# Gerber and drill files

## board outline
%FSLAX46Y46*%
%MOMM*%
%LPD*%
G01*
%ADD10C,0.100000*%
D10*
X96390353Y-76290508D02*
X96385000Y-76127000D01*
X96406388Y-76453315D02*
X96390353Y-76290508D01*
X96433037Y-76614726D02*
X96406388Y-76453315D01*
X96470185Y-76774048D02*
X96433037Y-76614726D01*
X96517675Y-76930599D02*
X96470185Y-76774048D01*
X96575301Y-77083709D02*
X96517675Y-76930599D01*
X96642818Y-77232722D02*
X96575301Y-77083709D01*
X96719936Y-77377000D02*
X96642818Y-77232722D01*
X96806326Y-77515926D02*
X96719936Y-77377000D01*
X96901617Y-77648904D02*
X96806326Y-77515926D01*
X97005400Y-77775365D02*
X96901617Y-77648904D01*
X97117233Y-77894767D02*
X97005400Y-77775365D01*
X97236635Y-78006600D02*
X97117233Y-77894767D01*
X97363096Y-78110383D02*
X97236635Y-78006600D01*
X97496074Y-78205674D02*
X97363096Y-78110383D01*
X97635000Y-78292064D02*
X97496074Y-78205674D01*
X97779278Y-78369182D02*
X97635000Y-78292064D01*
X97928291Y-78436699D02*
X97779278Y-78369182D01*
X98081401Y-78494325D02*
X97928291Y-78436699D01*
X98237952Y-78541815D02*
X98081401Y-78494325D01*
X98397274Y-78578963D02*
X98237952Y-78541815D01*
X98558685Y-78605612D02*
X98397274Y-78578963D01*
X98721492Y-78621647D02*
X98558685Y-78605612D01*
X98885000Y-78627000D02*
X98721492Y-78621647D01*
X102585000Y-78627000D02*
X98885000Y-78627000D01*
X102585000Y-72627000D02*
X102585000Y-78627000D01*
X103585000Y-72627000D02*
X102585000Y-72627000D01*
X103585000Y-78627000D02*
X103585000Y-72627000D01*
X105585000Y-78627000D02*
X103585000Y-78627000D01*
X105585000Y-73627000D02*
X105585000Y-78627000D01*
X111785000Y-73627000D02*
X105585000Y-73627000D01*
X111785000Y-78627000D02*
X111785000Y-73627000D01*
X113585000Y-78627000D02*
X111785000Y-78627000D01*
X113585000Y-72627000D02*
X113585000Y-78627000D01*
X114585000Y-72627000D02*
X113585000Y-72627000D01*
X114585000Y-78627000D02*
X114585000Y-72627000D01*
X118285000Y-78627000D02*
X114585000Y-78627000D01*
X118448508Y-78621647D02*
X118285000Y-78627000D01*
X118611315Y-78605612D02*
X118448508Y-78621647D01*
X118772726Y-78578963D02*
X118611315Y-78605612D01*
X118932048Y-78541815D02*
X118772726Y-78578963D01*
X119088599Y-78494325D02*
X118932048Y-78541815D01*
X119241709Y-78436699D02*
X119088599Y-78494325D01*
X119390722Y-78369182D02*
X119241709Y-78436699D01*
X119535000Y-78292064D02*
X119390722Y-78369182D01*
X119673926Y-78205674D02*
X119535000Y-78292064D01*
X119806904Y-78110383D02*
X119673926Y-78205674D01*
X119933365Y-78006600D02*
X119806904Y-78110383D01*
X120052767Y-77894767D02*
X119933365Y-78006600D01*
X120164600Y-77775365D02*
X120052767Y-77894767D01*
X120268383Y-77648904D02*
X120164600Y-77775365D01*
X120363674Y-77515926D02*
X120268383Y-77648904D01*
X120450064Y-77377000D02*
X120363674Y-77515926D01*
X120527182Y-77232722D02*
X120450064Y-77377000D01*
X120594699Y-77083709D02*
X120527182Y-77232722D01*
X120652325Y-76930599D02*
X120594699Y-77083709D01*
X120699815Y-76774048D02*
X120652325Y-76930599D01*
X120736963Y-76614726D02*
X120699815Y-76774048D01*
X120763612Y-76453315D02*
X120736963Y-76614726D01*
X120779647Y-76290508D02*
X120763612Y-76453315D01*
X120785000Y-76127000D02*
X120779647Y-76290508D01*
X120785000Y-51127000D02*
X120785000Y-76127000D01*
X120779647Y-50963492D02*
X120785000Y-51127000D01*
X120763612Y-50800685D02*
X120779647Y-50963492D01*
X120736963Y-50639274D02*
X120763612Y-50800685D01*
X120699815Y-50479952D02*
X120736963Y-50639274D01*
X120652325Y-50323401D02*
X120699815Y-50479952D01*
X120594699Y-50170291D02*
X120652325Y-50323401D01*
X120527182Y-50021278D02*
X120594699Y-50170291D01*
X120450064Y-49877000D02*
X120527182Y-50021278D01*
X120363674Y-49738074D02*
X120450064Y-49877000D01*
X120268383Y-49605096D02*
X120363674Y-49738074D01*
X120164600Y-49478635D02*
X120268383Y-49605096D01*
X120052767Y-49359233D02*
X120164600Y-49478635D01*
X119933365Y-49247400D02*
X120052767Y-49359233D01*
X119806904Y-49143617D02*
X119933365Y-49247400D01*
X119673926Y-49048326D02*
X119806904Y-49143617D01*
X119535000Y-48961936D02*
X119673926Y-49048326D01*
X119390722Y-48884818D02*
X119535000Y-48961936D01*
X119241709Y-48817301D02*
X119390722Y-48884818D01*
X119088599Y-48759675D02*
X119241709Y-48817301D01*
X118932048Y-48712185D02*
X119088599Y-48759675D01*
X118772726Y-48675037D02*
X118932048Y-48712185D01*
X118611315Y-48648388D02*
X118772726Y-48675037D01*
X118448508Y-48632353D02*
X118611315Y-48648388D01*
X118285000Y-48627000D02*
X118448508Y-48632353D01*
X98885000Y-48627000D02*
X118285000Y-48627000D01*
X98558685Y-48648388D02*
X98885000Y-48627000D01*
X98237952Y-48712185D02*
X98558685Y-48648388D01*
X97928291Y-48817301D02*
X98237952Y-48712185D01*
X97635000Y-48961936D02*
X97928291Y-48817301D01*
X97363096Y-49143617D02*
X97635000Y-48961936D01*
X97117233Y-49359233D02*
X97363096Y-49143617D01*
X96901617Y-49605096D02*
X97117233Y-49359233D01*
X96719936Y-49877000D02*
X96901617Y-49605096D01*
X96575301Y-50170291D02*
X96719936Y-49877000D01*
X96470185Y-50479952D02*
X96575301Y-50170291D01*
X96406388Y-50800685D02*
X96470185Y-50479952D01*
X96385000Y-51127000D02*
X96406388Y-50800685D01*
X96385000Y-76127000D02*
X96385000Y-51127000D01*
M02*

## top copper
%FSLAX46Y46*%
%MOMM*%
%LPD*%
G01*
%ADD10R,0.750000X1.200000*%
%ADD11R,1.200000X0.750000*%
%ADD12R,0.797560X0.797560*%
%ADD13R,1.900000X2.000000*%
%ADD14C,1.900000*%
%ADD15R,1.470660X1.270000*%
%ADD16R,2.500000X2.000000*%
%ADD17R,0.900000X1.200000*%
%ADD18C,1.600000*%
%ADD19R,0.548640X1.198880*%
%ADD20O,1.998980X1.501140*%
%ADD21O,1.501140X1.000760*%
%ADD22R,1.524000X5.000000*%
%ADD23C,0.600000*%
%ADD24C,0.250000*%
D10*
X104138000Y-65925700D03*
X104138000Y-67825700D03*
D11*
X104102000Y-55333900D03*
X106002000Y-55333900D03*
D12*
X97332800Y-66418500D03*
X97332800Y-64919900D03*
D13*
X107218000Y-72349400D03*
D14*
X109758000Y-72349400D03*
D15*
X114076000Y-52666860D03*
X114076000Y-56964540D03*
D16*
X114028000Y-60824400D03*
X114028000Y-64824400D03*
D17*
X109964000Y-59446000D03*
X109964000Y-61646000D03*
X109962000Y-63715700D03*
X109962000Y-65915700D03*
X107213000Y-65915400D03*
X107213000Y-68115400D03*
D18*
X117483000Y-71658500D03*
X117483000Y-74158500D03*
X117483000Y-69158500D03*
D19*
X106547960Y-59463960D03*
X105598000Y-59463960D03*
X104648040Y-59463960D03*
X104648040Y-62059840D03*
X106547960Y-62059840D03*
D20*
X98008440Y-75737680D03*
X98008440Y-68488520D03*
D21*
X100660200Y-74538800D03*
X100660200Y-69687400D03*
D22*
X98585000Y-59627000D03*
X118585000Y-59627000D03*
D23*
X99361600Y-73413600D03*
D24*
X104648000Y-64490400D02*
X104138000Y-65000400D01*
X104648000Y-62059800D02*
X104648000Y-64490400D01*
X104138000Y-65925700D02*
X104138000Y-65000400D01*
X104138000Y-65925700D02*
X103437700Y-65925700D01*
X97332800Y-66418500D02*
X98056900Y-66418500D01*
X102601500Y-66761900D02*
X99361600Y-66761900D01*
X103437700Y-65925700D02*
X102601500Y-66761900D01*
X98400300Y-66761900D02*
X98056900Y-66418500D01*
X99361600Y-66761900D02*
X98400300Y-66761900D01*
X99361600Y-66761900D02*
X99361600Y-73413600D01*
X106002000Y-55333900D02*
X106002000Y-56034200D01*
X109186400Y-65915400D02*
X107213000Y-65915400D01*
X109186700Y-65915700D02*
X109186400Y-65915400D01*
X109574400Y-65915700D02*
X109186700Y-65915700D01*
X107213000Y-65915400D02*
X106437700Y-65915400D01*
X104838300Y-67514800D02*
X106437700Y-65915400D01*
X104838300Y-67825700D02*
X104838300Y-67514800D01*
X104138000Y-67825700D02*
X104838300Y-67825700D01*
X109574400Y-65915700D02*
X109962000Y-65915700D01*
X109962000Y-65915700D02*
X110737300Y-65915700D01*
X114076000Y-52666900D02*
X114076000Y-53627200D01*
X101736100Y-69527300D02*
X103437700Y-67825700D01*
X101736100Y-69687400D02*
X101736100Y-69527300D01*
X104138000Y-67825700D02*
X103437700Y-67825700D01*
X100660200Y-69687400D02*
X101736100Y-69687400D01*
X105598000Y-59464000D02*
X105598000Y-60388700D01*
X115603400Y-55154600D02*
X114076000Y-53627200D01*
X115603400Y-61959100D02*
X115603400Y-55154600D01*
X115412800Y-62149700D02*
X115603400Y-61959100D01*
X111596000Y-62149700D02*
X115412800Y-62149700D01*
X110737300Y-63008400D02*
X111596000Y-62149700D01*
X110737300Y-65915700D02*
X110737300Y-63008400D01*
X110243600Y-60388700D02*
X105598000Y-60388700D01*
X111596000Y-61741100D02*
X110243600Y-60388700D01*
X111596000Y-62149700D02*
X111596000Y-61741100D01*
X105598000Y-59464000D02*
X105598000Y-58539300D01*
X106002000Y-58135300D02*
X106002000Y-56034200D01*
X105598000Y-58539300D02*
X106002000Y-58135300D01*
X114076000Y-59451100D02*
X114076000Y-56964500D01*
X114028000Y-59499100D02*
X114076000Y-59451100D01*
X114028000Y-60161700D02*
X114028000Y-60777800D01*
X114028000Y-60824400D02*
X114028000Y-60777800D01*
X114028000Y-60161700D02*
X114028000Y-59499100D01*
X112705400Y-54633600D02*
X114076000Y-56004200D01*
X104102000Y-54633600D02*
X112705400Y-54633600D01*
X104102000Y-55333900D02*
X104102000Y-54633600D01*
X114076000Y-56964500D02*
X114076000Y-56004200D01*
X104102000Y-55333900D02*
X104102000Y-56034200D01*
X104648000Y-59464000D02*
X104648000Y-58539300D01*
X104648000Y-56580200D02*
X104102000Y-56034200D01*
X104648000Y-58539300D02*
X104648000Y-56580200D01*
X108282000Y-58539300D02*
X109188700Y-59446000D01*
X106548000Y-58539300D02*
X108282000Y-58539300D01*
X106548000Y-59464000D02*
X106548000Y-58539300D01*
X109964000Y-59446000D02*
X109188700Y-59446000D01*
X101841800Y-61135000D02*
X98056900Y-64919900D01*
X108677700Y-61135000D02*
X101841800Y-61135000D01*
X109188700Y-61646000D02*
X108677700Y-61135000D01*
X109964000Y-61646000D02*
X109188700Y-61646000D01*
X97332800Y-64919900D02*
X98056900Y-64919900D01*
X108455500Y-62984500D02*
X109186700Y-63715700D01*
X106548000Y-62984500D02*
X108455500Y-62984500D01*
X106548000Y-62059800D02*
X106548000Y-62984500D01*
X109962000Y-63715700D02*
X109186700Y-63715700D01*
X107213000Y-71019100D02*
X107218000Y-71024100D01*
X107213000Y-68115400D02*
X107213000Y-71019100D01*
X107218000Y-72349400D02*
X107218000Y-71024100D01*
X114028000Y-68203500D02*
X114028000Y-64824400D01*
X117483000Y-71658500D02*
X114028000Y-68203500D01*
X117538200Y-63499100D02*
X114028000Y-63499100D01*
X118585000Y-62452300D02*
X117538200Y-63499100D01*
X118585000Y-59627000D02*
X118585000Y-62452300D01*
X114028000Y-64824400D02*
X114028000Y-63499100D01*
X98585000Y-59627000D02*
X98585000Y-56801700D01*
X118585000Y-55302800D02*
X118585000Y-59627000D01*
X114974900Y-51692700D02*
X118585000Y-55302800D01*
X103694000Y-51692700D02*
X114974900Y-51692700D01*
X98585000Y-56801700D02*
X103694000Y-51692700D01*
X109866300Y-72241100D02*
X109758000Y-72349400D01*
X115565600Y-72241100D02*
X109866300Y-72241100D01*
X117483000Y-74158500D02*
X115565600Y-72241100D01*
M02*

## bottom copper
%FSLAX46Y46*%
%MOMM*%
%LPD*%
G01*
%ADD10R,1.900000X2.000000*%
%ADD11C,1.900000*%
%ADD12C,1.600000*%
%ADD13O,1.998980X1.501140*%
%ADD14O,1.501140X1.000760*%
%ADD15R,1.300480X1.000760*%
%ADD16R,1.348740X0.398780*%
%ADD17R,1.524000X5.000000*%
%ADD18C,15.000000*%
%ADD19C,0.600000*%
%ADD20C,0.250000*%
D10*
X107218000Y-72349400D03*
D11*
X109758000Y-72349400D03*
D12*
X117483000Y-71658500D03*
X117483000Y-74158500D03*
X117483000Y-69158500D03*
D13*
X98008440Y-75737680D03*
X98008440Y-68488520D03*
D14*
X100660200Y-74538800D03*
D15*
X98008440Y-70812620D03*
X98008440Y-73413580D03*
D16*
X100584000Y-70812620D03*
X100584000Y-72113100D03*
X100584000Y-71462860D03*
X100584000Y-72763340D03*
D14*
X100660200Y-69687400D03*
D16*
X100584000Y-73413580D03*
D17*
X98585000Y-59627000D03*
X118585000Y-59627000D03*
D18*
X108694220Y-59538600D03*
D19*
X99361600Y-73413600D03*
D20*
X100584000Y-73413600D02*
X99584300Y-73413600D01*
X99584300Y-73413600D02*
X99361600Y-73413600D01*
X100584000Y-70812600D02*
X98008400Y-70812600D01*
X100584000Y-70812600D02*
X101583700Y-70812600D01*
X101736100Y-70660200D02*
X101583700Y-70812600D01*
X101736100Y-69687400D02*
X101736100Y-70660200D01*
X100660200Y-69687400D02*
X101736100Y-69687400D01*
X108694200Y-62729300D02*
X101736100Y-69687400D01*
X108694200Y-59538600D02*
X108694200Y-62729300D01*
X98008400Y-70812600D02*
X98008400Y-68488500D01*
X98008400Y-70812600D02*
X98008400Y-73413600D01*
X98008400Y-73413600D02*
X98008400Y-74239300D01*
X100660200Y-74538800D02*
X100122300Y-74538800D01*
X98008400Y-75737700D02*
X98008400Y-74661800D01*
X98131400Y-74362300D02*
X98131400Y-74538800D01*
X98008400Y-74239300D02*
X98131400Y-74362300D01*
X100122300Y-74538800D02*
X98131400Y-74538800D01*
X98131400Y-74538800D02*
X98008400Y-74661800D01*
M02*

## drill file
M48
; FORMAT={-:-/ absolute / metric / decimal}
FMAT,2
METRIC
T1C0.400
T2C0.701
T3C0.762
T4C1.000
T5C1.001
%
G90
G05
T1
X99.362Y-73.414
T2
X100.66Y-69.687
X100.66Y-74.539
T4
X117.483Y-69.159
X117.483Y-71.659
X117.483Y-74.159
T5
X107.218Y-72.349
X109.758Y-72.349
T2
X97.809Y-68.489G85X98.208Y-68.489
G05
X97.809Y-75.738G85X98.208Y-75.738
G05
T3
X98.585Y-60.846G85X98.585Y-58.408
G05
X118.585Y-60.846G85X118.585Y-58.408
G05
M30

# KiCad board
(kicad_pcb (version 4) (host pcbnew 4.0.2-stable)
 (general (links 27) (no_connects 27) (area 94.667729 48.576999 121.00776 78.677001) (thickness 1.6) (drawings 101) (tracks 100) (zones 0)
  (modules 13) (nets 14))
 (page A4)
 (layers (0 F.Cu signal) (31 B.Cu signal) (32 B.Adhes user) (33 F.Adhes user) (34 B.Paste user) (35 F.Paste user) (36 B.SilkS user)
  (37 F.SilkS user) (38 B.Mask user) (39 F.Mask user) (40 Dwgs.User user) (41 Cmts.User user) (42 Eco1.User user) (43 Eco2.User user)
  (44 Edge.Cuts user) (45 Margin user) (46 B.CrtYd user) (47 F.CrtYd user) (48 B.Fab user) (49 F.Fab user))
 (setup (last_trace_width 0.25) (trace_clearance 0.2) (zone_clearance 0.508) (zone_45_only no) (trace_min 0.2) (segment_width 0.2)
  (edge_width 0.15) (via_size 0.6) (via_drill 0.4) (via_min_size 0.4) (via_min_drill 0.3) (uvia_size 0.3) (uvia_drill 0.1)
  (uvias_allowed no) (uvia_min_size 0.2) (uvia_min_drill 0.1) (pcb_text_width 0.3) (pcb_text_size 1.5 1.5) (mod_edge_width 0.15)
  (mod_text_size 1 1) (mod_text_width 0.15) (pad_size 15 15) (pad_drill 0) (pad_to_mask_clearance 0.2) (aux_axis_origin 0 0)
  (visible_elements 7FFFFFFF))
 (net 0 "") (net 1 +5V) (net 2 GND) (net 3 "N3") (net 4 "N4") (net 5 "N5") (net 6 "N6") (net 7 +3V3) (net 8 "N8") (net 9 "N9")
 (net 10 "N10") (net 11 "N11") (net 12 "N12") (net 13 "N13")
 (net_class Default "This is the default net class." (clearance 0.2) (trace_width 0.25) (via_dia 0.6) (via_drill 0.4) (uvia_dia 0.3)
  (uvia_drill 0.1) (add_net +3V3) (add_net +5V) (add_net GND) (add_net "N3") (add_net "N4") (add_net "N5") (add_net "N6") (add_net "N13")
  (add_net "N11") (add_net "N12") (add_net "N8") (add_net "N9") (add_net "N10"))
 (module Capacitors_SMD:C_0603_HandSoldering (layer F.Cu) (at 104.138 66.8757 270)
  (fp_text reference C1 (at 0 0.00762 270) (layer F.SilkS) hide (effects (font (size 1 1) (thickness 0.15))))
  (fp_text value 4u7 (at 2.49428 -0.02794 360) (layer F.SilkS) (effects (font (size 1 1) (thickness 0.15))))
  (pad 1 smd rect (at -0.95 0 270) (size 1.2 0.75) (layers F.Cu F.Paste F.Mask) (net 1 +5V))
  (pad 2 smd rect (at 0.95 0 270) (size 1.2 0.75) (layers F.Cu F.Paste F.Mask) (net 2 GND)))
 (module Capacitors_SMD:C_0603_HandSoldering (layer F.Cu) (at 105.052 55.3339)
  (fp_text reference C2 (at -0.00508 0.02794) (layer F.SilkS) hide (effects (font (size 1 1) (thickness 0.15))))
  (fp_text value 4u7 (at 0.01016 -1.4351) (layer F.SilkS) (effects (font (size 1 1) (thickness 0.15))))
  (pad 1 smd rect (at -0.95 0) (size 1.2 0.75) (layers F.Cu F.Paste F.Mask) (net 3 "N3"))
  (pad 2 smd rect (at 0.95 0) (size 1.2 0.75) (layers F.Cu F.Paste F.Mask) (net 2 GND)))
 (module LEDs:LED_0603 (layer F.Cu) (at 97.3328 65.6692 270)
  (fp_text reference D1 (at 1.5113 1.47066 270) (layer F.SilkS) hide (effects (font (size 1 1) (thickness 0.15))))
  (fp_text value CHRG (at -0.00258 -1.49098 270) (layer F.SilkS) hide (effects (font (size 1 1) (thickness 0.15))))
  (pad 2 smd rect (at 0.7493 0 90) (size 0.79756 0.79756) (layers F.Cu F.Paste F.Mask) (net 1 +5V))
  (pad 1 smd rect (at -0.7493 0 90) (size 0.79756 0.79756) (layers F.Cu F.Paste F.Mask) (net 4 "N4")))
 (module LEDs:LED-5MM (layer F.Cu) (at 107.218 72.3494)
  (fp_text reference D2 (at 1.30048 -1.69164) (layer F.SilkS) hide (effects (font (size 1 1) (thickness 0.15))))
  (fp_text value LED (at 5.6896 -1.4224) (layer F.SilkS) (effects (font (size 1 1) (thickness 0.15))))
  (pad 1 thru_hole rect (at 0 0 90) (size 2 1.9) (drill 1.00076) (layers *.Cu *.Mask F.SilkS) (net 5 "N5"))
  (pad 2 thru_hole circle (at 2.54 0) (size 1.9 1.9) (drill 1.00076) (layers *.Cu *.Mask F.SilkS) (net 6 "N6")))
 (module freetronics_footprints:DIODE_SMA (layer F.Cu) (at 114.076 54.8157 270)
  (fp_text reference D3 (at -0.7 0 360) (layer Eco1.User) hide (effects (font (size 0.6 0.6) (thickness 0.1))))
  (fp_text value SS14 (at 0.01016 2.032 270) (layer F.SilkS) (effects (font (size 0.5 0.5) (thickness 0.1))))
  (pad A smd rect (at -2.14884 0 270) (size 1.27 1.47066) (layers F.Cu F.Paste F.Mask) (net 2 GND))
  (pad K smd rect (at 2.14884 0 270) (size 1.27 1.47066) (layers F.Cu F.Paste F.Mask) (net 3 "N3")))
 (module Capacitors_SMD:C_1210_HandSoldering (layer F.Cu) (at 114.028 62.8244 270)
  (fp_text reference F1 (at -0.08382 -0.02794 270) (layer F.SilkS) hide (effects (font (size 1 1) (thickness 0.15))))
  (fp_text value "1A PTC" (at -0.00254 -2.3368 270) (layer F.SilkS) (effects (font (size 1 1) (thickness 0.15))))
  (pad 1 smd rect (at -2 0 270) (size 2 2.5) (layers F.Cu F.Paste F.Mask) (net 3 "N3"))
  (pad 2 smd rect (at 2 0 270) (size 2 2.5) (layers F.Cu F.Paste F.Mask) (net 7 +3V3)))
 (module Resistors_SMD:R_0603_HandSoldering (layer F.Cu) (at 109.964 60.546 270)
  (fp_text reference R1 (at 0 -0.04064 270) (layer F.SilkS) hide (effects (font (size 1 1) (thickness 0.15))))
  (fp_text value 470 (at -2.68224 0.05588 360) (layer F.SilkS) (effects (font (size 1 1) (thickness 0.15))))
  (pad 1 smd rect (at -1.1 0 270) (size 1.2 0.9) (layers F.Cu F.Paste F.Mask) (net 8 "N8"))
  (pad 2 smd rect (at 1.1 0 270) (size 1.2 0.9) (layers F.Cu F.Paste F.Mask) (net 4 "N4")))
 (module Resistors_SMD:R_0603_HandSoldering (layer F.Cu) (at 109.962 64.8157 270)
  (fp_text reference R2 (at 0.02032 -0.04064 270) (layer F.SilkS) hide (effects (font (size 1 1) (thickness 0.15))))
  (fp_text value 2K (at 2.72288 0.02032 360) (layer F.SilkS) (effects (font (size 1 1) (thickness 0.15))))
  (pad 1 smd rect (at -1.1 0 270) (size 1.2 0.9) (layers F.Cu F.Paste F.Mask) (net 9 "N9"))
  (pad 2 smd rect (at 1.1 0 270) (size 1.2 0.9) (layers F.Cu F.Paste F.Mask) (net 2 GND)))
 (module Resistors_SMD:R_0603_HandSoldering (layer F.Cu) (at 107.213 67.0154 270)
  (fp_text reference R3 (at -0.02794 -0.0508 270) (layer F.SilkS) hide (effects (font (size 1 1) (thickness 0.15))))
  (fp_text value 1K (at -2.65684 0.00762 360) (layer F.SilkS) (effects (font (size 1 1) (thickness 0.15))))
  (pad 1 smd rect (at -1.1 0 270) (size 1.2 0.9) (layers F.Cu F.Paste F.Mask) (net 2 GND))
  (pad 2 smd rect (at 1.1 0 270) (size 1.2 0.9) (layers F.Cu F.Paste F.Mask) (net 5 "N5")))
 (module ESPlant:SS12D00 (layer F.Cu) (at 117.483 71.6585 90)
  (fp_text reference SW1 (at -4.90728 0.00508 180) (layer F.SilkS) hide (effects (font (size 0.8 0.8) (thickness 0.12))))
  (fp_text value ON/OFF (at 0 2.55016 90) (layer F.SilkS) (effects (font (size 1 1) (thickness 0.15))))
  (pad 2 thru_hole circle (at 0 0 90) (size 1.6 1.6) (drill 1) (layers *.Cu *.Mask F.SilkS) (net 7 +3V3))
  (pad 1 thru_hole circle (at -2.5 0 90) (size 1.6 1.6) (drill 1) (layers *.Cu *.Mask F.SilkS) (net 6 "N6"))
  (pad 3 thru_hole circle (at 2.5 0 90) (size 1.6 1.6) (drill 1) (layers *.Cu *.Mask F.SilkS) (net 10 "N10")))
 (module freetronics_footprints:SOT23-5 (layer F.Cu) (at 105.598 60.7619 180)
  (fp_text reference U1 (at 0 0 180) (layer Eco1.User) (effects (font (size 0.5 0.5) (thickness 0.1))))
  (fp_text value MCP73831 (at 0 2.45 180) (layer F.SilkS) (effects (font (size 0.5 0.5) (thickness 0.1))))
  (pad 1 smd rect (at -0.94996 1.29794 180) (size 0.54864 1.19888) (layers F.Cu F.Paste F.Mask) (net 8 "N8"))
  (pad 2 smd rect (at 0 1.29794 180) (size 0.54864 1.19888) (layers F.Cu F.Paste F.Mask) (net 2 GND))
  (pad 3 smd rect (at 0.94996 1.29794 180) (size 0.54864 1.19888) (layers F.Cu F.Paste F.Mask) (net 3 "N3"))
  (pad 4 smd rect (at 0.94996 -1.29794 180) (size 0.54864 1.19888) (layers F.Cu F.Paste F.Mask) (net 1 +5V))
  (pad 5 smd rect (at -0.94996 -1.29794 180) (size 0.54864 1.19888) (layers F.Cu F.Paste F.Mask) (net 9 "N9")))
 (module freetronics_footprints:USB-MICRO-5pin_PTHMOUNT (layer B.Cu) (at 100.584 72.1131)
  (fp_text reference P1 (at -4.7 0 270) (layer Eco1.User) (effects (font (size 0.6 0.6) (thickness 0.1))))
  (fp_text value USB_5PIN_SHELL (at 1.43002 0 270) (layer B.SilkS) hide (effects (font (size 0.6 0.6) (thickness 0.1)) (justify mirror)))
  (pad SHLD thru_hole oval (at -2.57556 3.62458) (size 1.99898 1.50114) (drill oval 1.09982 0.70104) (layers *.Cu *.Mask B.SilkS)
   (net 2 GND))
  (pad SHLD thru_hole oval (at -2.57556 -3.62458) (size 1.99898 1.50114) (drill oval 1.09982 0.70104) (layers *.Cu *.Mask B.SilkS)
   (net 2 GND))
  (pad SHLD thru_hole oval (at 0.0762 2.4257) (size 1.50114 1.00076) (drill 0.70104) (layers *.Cu *.Mask B.SilkS) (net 2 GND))
  (pad SHLD smd rect (at -2.57556 -1.30048) (size 1.30048 1.00076) (layers B.Cu B.Paste B.Mask) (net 2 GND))
  (pad SHLD smd rect (at -2.57556 1.30048) (size 1.30048 1.00076) (layers B.Cu B.Paste B.Mask) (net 2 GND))
  (pad 5 smd rect (at 0 -1.30048) (size 1.34874 0.39878) (layers B.Cu B.Paste B.Mask) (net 2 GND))
  (pad 3 smd rect (at 0 0) (size 1.34874 0.39878) (layers B.Cu B.Paste B.Mask) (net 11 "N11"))
  (pad 4 smd rect (at 0 -0.65024) (size 1.34874 0.39878) (layers B.Cu B.Paste B.Mask) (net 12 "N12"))
  (pad 2 smd rect (at 0 0.65024) (size 1.34874 0.39878) (layers B.Cu B.Paste B.Mask) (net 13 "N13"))
  (pad SHLD thru_hole oval (at 0.0762 -2.4257) (size 1.50114 1.00076) (drill 0.70104) (layers *.Cu *.Mask B.SilkS) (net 2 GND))
  (pad 1 smd rect (at 0 1.30048) (size 1.34874 0.39878) (layers B.Cu B.Paste B.Mask) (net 1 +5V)))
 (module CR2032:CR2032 (layer B.Cu) (at 108.585 59.627 180)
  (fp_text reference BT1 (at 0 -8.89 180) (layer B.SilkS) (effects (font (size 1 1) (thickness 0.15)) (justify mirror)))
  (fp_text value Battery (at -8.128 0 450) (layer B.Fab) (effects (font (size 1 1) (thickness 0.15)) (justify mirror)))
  (pad 1 thru_hole rect (at 10 0 180) (size 1.524 5) (drill oval 0.762 3.2) (layers *.Cu *.Mask B.SilkS) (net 7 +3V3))
  (pad 1 thru_hole rect (at -10 0 180) (size 1.524 5) (drill oval 0.762 3.2) (layers *.Cu *.Mask B.SilkS) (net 7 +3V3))
  (pad 2 smd circle (at -0.10922 0.0884 180) (size 15 15) (layers B.Cu B.Paste B.Mask) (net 2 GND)))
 (gr_line (start 96.390353 76.290508) (end 96.385 76.127) (layer Edge.Cuts) (width 0.1))
 (gr_line (start 96.406388 76.453315) (end 96.390353 76.290508) (layer Edge.Cuts) (width 0.1))
 (gr_line (start 96.433037 76.614726) (end 96.406388 76.453315) (layer Edge.Cuts) (width 0.1))
 (gr_line (start 96.470185 76.774048) (end 96.433037 76.614726) (layer Edge.Cuts) (width 0.1))
 (gr_line (start 96.517675 76.930599) (end 96.470185 76.774048) (layer Edge.Cuts) (width 0.1))
 (gr_line (start 96.575301 77.083709) (end 96.517675 76.930599) (layer Edge.Cuts) (width 0.1))
 (gr_line (start 96.642818 77.232722) (end 96.575301 77.083709) (layer Edge.Cuts) (width 0.1))
 (gr_line (start 96.719936 77.377) (end 96.642818 77.232722) (layer Edge.Cuts) (width 0.1))
 (gr_line (start 96.806326 77.515926) (end 96.719936 77.377) (layer Edge.Cuts) (width 0.1))
 (gr_line (start 96.901617 77.648904) (end 96.806326 77.515926) (layer Edge.Cuts) (width 0.1))
 (gr_line (start 97.0054 77.775365) (end 96.901617 77.648904) (layer Edge.Cuts) (width 0.1))
 (gr_line (start 97.117233 77.894767) (end 97.0054 77.775365) (layer Edge.Cuts) (width 0.1))
 (gr_line (start 97.236635 78.0066) (end 97.117233 77.894767) (layer Edge.Cuts) (width 0.1))
 (gr_line (start 97.363096 78.110383) (end 97.236635 78.0066) (layer Edge.Cuts) (width 0.1))
 (gr_line (start 97.496074 78.205674) (end 97.363096 78.110383) (layer Edge.Cuts) (width 0.1))
 (gr_line (start 97.635 78.292064) (end 97.496074 78.205674) (layer Edge.Cuts) (width 0.1))
 (gr_line (start 97.779278 78.369182) (end 97.635 78.292064) (layer Edge.Cuts) (width 0.1))
 (gr_line (start 97.928291 78.436699) (end 97.779278 78.369182) (layer Edge.Cuts) (width 0.1))
 (gr_line (start 98.081401 78.494325) (end 97.928291 78.436699) (layer Edge.Cuts) (width 0.1))
 (gr_line (start 98.237952 78.541815) (end 98.081401 78.494325) (layer Edge.Cuts) (width 0.1))
 (gr_line (start 98.397274 78.578963) (end 98.237952 78.541815) (layer Edge.Cuts) (width 0.1))
 (gr_line (start 98.558685 78.605612) (end 98.397274 78.578963) (layer Edge.Cuts) (width 0.1))
 (gr_line (start 98.721492 78.621647) (end 98.558685 78.605612) (layer Edge.Cuts) (width 0.1))
 (gr_line (start 98.885 78.627) (end 98.721492 78.621647) (layer Edge.Cuts) (width 0.1))
 (gr_line (start 102.585 78.627) (end 98.885 78.627) (layer Edge.Cuts) (width 0.1))
 (gr_line (start 102.585 72.627) (end 102.585 78.627) (layer Edge.Cuts) (width 0.1))
 (gr_line (start 103.585 72.627) (end 102.585 72.627) (layer Edge.Cuts) (width 0.1))
 (gr_line (start 103.585 78.627) (end 103.585 72.627) (layer Edge.Cuts) (width 0.1))
 (gr_line (start 105.585 78.627) (end 103.585 78.627) (layer Edge.Cuts) (width 0.1))
 (gr_line (start 105.585 73.627) (end 105.585 78.627) (layer Edge.Cuts) (width 0.1))
 (gr_line (start 111.785 73.627) (end 105.585 73.627) (layer Edge.Cuts) (width 0.1))
 (gr_line (start 111.785 78.627) (end 111.785 73.627) (layer Edge.Cuts) (width 0.1))
 (gr_line (start 113.585 78.627) (end 111.785 78.627) (layer Edge.Cuts) (width 0.1))
 (gr_line (start 113.585 72.627) (end 113.585 78.627) (layer Edge.Cuts) (width 0.1))
 (gr_line (start 114.585 72.627) (end 113.585 72.627) (layer Edge.Cuts) (width 0.1))
 (gr_line (start 114.585 78.627) (end 114.585 72.627) (layer Edge.Cuts) (width 0.1))
 (gr_line (start 118.285 78.627) (end 114.585 78.627) (layer Edge.Cuts) (width 0.1))
 (gr_line (start 118.448508 78.621647) (end 118.285 78.627) (layer Edge.Cuts) (width 0.1))
 (gr_line (start 118.611315 78.605612) (end 118.448508 78.621647) (layer Edge.Cuts) (width 0.1))
 (gr_line (start 118.772726 78.578963) (end 118.611315 78.605612) (layer Edge.Cuts) (width 0.1))
 (gr_line (start 118.932048 78.541815) (end 118.772726 78.578963) (layer Edge.Cuts) (width 0.1))
 (gr_line (start 119.088599 78.494325) (end 118.932048 78.541815) (layer Edge.Cuts) (width 0.1))
 (gr_line (start 119.241709 78.436699) (end 119.088599 78.494325) (layer Edge.Cuts) (width 0.1))
 (gr_line (start 119.390722 78.369182) (end 119.241709 78.436699) (layer Edge.Cuts) (width 0.1))
 (gr_line (start 119.535 78.292064) (end 119.390722 78.369182) (layer Edge.Cuts) (width 0.1))
 (gr_line (start 119.673926 78.205674) (end 119.535 78.292064) (layer Edge.Cuts) (width 0.1))
 (gr_line (start 119.806904 78.110383) (end 119.673926 78.205674) (layer Edge.Cuts) (width 0.1))
 (gr_line (start 119.933365 78.0066) (end 119.806904 78.110383) (layer Edge.Cuts) (width 0.1))
 (gr_line (start 120.052767 77.894767) (end 119.933365 78.0066) (layer Edge.Cuts) (width 0.1))
 (gr_line (start 120.1646 77.775365) (end 120.052767 77.894767) (layer Edge.Cuts) (width 0.1))
 (gr_line (start 120.268383 77.648904) (end 120.1646 77.775365) (layer Edge.Cuts) (width 0.1))
 (gr_line (start 120.363674 77.515926) (end 120.268383 77.648904) (layer Edge.Cuts) (width 0.1))
 (gr_line (start 120.450064 77.377) (end 120.363674 77.515926) (layer Edge.Cuts) (width 0.1))
 (gr_line (start 120.527182 77.232722) (end 120.450064 77.377) (layer Edge.Cuts) (width 0.1))
 (gr_line (start 120.594699 77.083709) (end 120.527182 77.232722) (layer Edge.Cuts) (width 0.1))
 (gr_line (start 120.652325 76.930599) (end 120.594699 77.083709) (layer Edge.Cuts) (width 0.1))
 (gr_line (start 120.699815 76.774048) (end 120.652325 76.930599) (layer Edge.Cuts) (width 0.1))
 (gr_line (start 120.736963 76.614726) (end 120.699815 76.774048) (layer Edge.Cuts) (width 0.1))
 (gr_line (start 120.763612 76.453315) (end 120.736963 76.614726) (layer Edge.Cuts) (width 0.1))
 (gr_line (start 120.779647 76.290508) (end 120.763612 76.453315) (layer Edge.Cuts) (width 0.1))
 (gr_line (start 120.785 76.127) (end 120.779647 76.290508) (layer Edge.Cuts) (width 0.1))
 (gr_line (start 120.785 51.127) (end 120.785 76.127) (layer Edge.Cuts) (width 0.1))
 (gr_line (start 120.779647 50.963492) (end 120.785 51.127) (layer Edge.Cuts) (width 0.1))
 (gr_line (start 120.763612 50.800685) (end 120.779647 50.963492) (layer Edge.Cuts) (width 0.1))
 (gr_line (start 120.736963 50.639274) (end 120.763612 50.800685) (layer Edge.Cuts) (width 0.1))
 (gr_line (start 120.699815 50.479952) (end 120.736963 50.639274) (layer Edge.Cuts) (width 0.1))
 (gr_line (start 120.652325 50.323401) (end 120.699815 50.479952) (layer Edge.Cuts) (width 0.1))
 (gr_line (start 120.594699 50.170291) (end 120.652325 50.323401) (layer Edge.Cuts) (width 0.1))
 (gr_line (start 120.527182 50.021278) (end 120.594699 50.170291) (layer Edge.Cuts) (width 0.1))
 (gr_line (start 120.450064 49.877) (end 120.527182 50.021278) (layer Edge.Cuts) (width 0.1))
 (gr_line (start 120.363674 49.738074) (end 120.450064 49.877) (layer Edge.Cuts) (width 0.1))
 (gr_line (start 120.268383 49.605096) (end 120.363674 49.738074) (layer Edge.Cuts) (width 0.1))
 (gr_line (start 120.1646 49.478635) (end 120.268383 49.605096) (layer Edge.Cuts) (width 0.1))
 (gr_line (start 120.052767 49.359233) (end 120.1646 49.478635) (layer Edge.Cuts) (width 0.1))
 (gr_line (start 119.933365 49.2474) (end 120.052767 49.359233) (layer Edge.Cuts) (width 0.1))
 (gr_line (start 119.806904 49.143617) (end 119.933365 49.2474) (layer Edge.Cuts) (width 0.1))
 (gr_line (start 119.673926 49.048326) (end 119.806904 49.143617) (layer Edge.Cuts) (width 0.1))
 (gr_line (start 119.535 48.961936) (end 119.673926 49.048326) (layer Edge.Cuts) (width 0.1))
 (gr_line (start 119.390722 48.884818) (end 119.535 48.961936) (layer Edge.Cuts) (width 0.1))
 (gr_line (start 119.241709 48.817301) (end 119.390722 48.884818) (layer Edge.Cuts) (width 0.1))
 (gr_line (start 119.088599 48.759675) (end 119.241709 48.817301) (layer Edge.Cuts) (width 0.1))
 (gr_line (start 118.932048 48.712185) (end 119.088599 48.759675) (layer Edge.Cuts) (width 0.1))
 (gr_line (start 118.772726 48.675037) (end 118.932048 48.712185) (layer Edge.Cuts) (width 0.1))
 (gr_line (start 118.611315 48.648388) (end 118.772726 48.675037) (layer Edge.Cuts) (width 0.1))
 (gr_line (start 118.448508 48.632353) (end 118.611315 48.648388) (layer Edge.Cuts) (width 0.1))
 (gr_line (start 118.285 48.627) (end 118.448508 48.632353) (layer Edge.Cuts) (width 0.1))
 (gr_line (start 98.885 48.627) (end 118.285 48.627) (layer Edge.Cuts) (width 0.1))
 (gr_line (start 98.558685 48.648388) (end 98.885 48.627) (layer Edge.Cuts) (width 0.1))
 (gr_line (start 98.237952 48.712185) (end 98.558685 48.648388) (layer Edge.Cuts) (width 0.1))
 (gr_line (start 97.928291 48.817301) (end 98.237952 48.712185) (layer Edge.Cuts) (width 0.1))
 (gr_line (start 97.635 48.961936) (end 97.928291 48.817301) (layer Edge.Cuts) (width 0.1))
 (gr_line (start 97.363096 49.143617) (end 97.635 48.961936) (layer Edge.Cuts) (width 0.1))
 (gr_line (start 97.117233 49.359233) (end 97.363096 49.143617) (layer Edge.Cuts) (width 0.1))
 (gr_line (start 96.901617 49.605096) (end 97.117233 49.359233) (layer Edge.Cuts) (width 0.1))
 (gr_line (start 96.719936 49.877) (end 96.901617 49.605096) (layer Edge.Cuts) (width 0.1))
 (gr_line (start 96.575301 50.170291) (end 96.719936 49.877) (layer Edge.Cuts) (width 0.1))
 (gr_line (start 96.470185 50.479952) (end 96.575301 50.170291) (layer Edge.Cuts) (width 0.1))
 (gr_line (start 96.406388 50.800685) (end 96.470185 50.479952) (layer Edge.Cuts) (width 0.1))
 (gr_line (start 96.385 51.127) (end 96.406388 50.800685) (layer Edge.Cuts) (width 0.1))
 (gr_line (start 96.385 76.127) (end 96.385 51.127) (layer Edge.Cuts) (width 0.1))
 (via (at 99.3616 73.4136) (size 0.6) (layers F.Cu B.Cu) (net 1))
 (segment (start 104.648 64.4904) (end 104.138 65.0004) (width 0.25) (layer F.Cu) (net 1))
 (segment (start 104.648 62.0598) (end 104.648 64.4904) (width 0.25) (layer F.Cu) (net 1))
 (segment (start 104.138 65.9257) (end 104.138 65.0004) (width 0.25) (layer F.Cu) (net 1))
 (segment (start 104.138 65.9257) (end 103.4377 65.9257) (width 0.25) (layer F.Cu) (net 1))
 (segment (start 97.3328 66.4185) (end 98.0569 66.4185) (width 0.25) (layer F.Cu) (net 1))
 (segment (start 102.6015 66.7619) (end 99.3616 66.7619) (width 0.25) (layer F.Cu) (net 1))
 (segment (start 103.4377 65.9257) (end 102.6015 66.7619) (width 0.25) (layer F.Cu) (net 1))
 (segment (start 98.4003 66.7619) (end 98.0569 66.4185) (width 0.25) (layer F.Cu) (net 1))
 (segment (start 99.3616 66.7619) (end 98.4003 66.7619) (width 0.25) (layer F.Cu) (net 1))
 (segment (start 100.584 73.4136) (end 99.5843 73.4136) (width 0.25) (layer B.Cu) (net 1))
 (segment (start 99.5843 73.4136) (end 99.3616 73.4136) (width 0.25) (layer B.Cu) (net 1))
 (segment (start 99.3616 66.7619) (end 99.3616 73.4136) (width 0.25) (layer F.Cu) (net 1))
 (segment (start 100.584 70.8126) (end 98.0084 70.8126) (width 0.25) (layer B.Cu) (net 2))
 (segment (start 106.002 55.3339) (end 106.002 56.0342) (width 0.25) (layer F.Cu) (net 2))
 (segment (start 109.1864 65.9154) (end 107.213 65.9154) (width 0.25) (layer F.Cu) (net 2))
 (segment (start 109.1867 65.9157) (end 109.1864 65.9154) (width 0.25) (layer F.Cu) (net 2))
 (segment (start 109.5744 65.9157) (end 109.1867 65.9157) (width 0.25) (layer F.Cu) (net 2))
 (segment (start 100.584 70.8126) (end 101.5837 70.8126) (width 0.25) (layer B.Cu) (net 2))
 (segment (start 101.7361 70.6602) (end 101.5837 70.8126) (width 0.25) (layer B.Cu) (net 2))
 (segment (start 101.7361 69.6874) (end 101.7361 70.6602) (width 0.25) (layer B.Cu) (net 2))
 (segment (start 100.6602 69.6874) (end 101.7361 69.6874) (width 0.25) (layer B.Cu) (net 2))
 (segment (start 107.213 65.9154) (end 106.4377 65.9154) (width 0.25) (layer F.Cu) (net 2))
 (segment (start 104.8383 67.5148) (end 106.4377 65.9154) (width 0.25) (layer F.Cu) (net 2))
 (segment (start 104.8383 67.8257) (end 104.8383 67.5148) (width 0.25) (layer F.Cu) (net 2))
 (segment (start 104.138 67.8257) (end 104.8383 67.8257) (width 0.25) (layer F.Cu) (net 2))
 (segment (start 109.5744 65.9157) (end 109.962 65.9157) (width 0.25) (layer F.Cu) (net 2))
 (segment (start 109.962 65.9157) (end 110.7373 65.9157) (width 0.25) (layer F.Cu) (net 2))
 (segment (start 114.076 52.6669) (end 114.076 53.6272) (width 0.25) (layer F.Cu) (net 2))
 (segment (start 108.6942 62.7293) (end 101.7361 69.6874) (width 0.25) (layer B.Cu) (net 2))
 (segment (start 108.6942 59.5386) (end 108.6942 62.7293) (width 0.25) (layer B.Cu) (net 2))
 (segment (start 98.0084 70.8126) (end 98.0084 68.4885) (width 0.25) (layer B.Cu) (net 2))
 (segment (start 98.0084 70.8126) (end 98.0084 73.4136) (width 0.25) (layer B.Cu) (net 2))
 (segment (start 98.0084 73.4136) (end 98.0084 74.2393) (width 0.25) (layer B.Cu) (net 2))
 (segment (start 100.6602 74.5388) (end 100.1223 74.5388) (width 0.25) (layer B.Cu) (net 2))
 (segment (start 98.0084 75.7377) (end 98.0084 74.6618) (width 0.25) (layer B.Cu) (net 2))
 (segment (start 98.1314 74.3623) (end 98.1314 74.5388) (width 0.25) (layer B.Cu) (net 2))
 (segment (start 98.0084 74.2393) (end 98.1314 74.3623) (width 0.25) (layer B.Cu) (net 2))
 (segment (start 100.1223 74.5388) (end 98.1314 74.5388) (width 0.25) (layer B.Cu) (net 2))
 (segment (start 98.1314 74.5388) (end 98.0084 74.6618) (width 0.25) (layer B.Cu) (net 2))
 (segment (start 101.7361 69.5273) (end 103.4377 67.8257) (width 0.25) (layer F.Cu) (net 2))
 (segment (start 101.7361 69.6874) (end 101.7361 69.5273) (width 0.25) (layer F.Cu) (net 2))
 (segment (start 104.138 67.8257) (end 103.4377 67.8257) (width 0.25) (layer F.Cu) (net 2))
 (segment (start 100.6602 69.6874) (end 101.7361 69.6874) (width 0.25) (layer F.Cu) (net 2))
 (segment (start 105.598 59.464) (end 105.598 60.3887) (width 0.25) (layer F.Cu) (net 2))
 (segment (start 115.6034 55.1546) (end 114.076 53.6272) (width 0.25) (layer F.Cu) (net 2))
 (segment (start 115.6034 61.9591) (end 115.6034 55.1546) (width 0.25) (layer F.Cu) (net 2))
 (segment (start 115.4128 62.1497) (end 115.6034 61.9591) (width 0.25) (layer F.Cu) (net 2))
 (segment (start 111.596 62.1497) (end 115.4128 62.1497) (width 0.25) (layer F.Cu) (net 2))
 (segment (start 110.7373 63.0084) (end 111.596 62.1497) (width 0.25) (layer F.Cu) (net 2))
 (segment (start 110.7373 65.9157) (end 110.7373 63.0084) (width 0.25) (layer F.Cu) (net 2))
 (segment (start 110.2436 60.3887) (end 105.598 60.3887) (width 0.25) (layer F.Cu) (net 2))
 (segment (start 111.596 61.7411) (end 110.2436 60.3887) (width 0.25) (layer F.Cu) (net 2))
 (segment (start 111.596 62.1497) (end 111.596 61.7411) (width 0.25) (layer F.Cu) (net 2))
 (segment (start 105.598 59.464) (end 105.598 58.5393) (width 0.25) (layer F.Cu) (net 2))
 (segment (start 106.002 58.1353) (end 106.002 56.0342) (width 0.25) (layer F.Cu) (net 2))
 (segment (start 105.598 58.5393) (end 106.002 58.1353) (width 0.25) (layer F.Cu) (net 2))
 (segment (start 114.076 59.4511) (end 114.076 56.9645) (width 0.25) (layer F.Cu) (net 3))
 (segment (start 114.028 59.4991) (end 114.076 59.4511) (width 0.25) (layer F.Cu) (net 3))
 (segment (start 114.028 60.1617) (end 114.028 60.7778) (width 0.25) (layer F.Cu) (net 3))
 (segment (start 114.028 60.8244) (end 114.028 60.7778) (width 0.25) (layer F.Cu) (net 3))
 (segment (start 114.028 60.1617) (end 114.028 59.4991) (width 0.25) (layer F.Cu) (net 3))
 (segment (start 112.7054 54.6336) (end 114.076 56.0042) (width 0.25) (layer F.Cu) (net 3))
 (segment (start 104.102 54.6336) (end 112.7054 54.6336) (width 0.25) (layer F.Cu) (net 3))
 (segment (start 104.102 55.3339) (end 104.102 54.6336) (width 0.25) (layer F.Cu) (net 3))
 (segment (start 114.076 56.9645) (end 114.076 56.0042) (width 0.25) (layer F.Cu) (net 3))
 (segment (start 104.102 55.3339) (end 104.102 56.0342) (width 0.25) (layer F.Cu) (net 3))
 (segment (start 104.648 59.464) (end 104.648 58.5393) (width 0.25) (layer F.Cu) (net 3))
 (segment (start 104.648 56.5802) (end 104.102 56.0342) (width 0.25) (layer F.Cu) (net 3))
 (segment (start 104.648 58.5393) (end 104.648 56.5802) (width 0.25) (layer F.Cu) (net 3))
 (segment (start 108.282 58.5393) (end 109.1887 59.446) (width 0.25) (layer F.Cu) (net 8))
 (segment (start 106.548 58.5393) (end 108.282 58.5393) (width 0.25) (layer F.Cu) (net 8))
 (segment (start 106.548 59.464) (end 106.548 58.5393) (width 0.25) (layer F.Cu) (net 8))
 (segment (start 109.964 59.446) (end 109.1887 59.446) (width 0.25) (layer F.Cu) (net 8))
 (segment (start 101.8418 61.135) (end 98.0569 64.9199) (width 0.25) (layer F.Cu) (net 4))
 (segment (start 108.6777 61.135) (end 101.8418 61.135) (width 0.25) (layer F.Cu) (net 4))
 (segment (start 109.1887 61.646) (end 108.6777 61.135) (width 0.25) (layer F.Cu) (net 4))
 (segment (start 109.964 61.646) (end 109.1887 61.646) (width 0.25) (layer F.Cu) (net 4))
 (segment (start 97.3328 64.9199) (end 98.0569 64.9199) (width 0.25) (layer F.Cu) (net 4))
 (segment (start 108.4555 62.9845) (end 109.1867 63.7157) (width 0.25) (layer F.Cu) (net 9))
 (segment (start 106.548 62.9845) (end 108.4555 62.9845) (width 0.25) (layer F.Cu) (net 9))
 (segment (start 106.548 62.0598) (end 106.548 62.9845) (width 0.25) (layer F.Cu) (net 9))
 (segment (start 109.962 63.7157) (end 109.1867 63.7157) (width 0.25) (layer F.Cu) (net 9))
 (segment (start 107.213 71.0191) (end 107.218 71.0241) (width 0.25) (layer F.Cu) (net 5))
 (segment (start 107.213 68.1154) (end 107.213 71.0191) (width 0.25) (layer F.Cu) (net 5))
 (segment (start 107.218 72.3494) (end 107.218 71.0241) (width 0.25) (layer F.Cu) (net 5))
 (segment (start 114.028 68.2035) (end 114.028 64.8244) (width 0.25) (layer F.Cu) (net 7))
 (segment (start 117.483 71.6585) (end 114.028 68.2035) (width 0.25) (layer F.Cu) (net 7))
 (segment (start 117.5382 63.4991) (end 114.028 63.4991) (width 0.25) (layer F.Cu) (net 7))
 (segment (start 118.585 62.4523) (end 117.5382 63.4991) (width 0.25) (layer F.Cu) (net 7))
 (segment (start 118.585 59.627) (end 118.585 62.4523) (width 0.25) (layer F.Cu) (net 7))
 (segment (start 114.028 64.8244) (end 114.028 63.4991) (width 0.25) (layer F.Cu) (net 7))
 (segment (start 98.585 59.627) (end 98.585 56.8017) (width 0.25) (layer F.Cu) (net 7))
 (segment (start 118.585 55.3028) (end 118.585 59.627) (width 0.25) (layer F.Cu) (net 7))
 (segment (start 114.9749 51.6927) (end 118.585 55.3028) (width 0.25) (layer F.Cu) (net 7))
 (segment (start 103.694 51.6927) (end 114.9749 51.6927) (width 0.25) (layer F.Cu) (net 7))
 (segment (start 98.585 56.8017) (end 103.694 51.6927) (width 0.25) (layer F.Cu) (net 7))
 (segment (start 109.8663 72.2411) (end 109.758 72.3494) (width 0.25) (layer F.Cu) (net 6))
 (segment (start 115.5656 72.2411) (end 109.8663 72.2411) (width 0.25) (layer F.Cu) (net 6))
 (segment (start 117.483 74.1585) (end 115.5656 72.2411) (width 0.25) (layer F.Cu) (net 6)))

